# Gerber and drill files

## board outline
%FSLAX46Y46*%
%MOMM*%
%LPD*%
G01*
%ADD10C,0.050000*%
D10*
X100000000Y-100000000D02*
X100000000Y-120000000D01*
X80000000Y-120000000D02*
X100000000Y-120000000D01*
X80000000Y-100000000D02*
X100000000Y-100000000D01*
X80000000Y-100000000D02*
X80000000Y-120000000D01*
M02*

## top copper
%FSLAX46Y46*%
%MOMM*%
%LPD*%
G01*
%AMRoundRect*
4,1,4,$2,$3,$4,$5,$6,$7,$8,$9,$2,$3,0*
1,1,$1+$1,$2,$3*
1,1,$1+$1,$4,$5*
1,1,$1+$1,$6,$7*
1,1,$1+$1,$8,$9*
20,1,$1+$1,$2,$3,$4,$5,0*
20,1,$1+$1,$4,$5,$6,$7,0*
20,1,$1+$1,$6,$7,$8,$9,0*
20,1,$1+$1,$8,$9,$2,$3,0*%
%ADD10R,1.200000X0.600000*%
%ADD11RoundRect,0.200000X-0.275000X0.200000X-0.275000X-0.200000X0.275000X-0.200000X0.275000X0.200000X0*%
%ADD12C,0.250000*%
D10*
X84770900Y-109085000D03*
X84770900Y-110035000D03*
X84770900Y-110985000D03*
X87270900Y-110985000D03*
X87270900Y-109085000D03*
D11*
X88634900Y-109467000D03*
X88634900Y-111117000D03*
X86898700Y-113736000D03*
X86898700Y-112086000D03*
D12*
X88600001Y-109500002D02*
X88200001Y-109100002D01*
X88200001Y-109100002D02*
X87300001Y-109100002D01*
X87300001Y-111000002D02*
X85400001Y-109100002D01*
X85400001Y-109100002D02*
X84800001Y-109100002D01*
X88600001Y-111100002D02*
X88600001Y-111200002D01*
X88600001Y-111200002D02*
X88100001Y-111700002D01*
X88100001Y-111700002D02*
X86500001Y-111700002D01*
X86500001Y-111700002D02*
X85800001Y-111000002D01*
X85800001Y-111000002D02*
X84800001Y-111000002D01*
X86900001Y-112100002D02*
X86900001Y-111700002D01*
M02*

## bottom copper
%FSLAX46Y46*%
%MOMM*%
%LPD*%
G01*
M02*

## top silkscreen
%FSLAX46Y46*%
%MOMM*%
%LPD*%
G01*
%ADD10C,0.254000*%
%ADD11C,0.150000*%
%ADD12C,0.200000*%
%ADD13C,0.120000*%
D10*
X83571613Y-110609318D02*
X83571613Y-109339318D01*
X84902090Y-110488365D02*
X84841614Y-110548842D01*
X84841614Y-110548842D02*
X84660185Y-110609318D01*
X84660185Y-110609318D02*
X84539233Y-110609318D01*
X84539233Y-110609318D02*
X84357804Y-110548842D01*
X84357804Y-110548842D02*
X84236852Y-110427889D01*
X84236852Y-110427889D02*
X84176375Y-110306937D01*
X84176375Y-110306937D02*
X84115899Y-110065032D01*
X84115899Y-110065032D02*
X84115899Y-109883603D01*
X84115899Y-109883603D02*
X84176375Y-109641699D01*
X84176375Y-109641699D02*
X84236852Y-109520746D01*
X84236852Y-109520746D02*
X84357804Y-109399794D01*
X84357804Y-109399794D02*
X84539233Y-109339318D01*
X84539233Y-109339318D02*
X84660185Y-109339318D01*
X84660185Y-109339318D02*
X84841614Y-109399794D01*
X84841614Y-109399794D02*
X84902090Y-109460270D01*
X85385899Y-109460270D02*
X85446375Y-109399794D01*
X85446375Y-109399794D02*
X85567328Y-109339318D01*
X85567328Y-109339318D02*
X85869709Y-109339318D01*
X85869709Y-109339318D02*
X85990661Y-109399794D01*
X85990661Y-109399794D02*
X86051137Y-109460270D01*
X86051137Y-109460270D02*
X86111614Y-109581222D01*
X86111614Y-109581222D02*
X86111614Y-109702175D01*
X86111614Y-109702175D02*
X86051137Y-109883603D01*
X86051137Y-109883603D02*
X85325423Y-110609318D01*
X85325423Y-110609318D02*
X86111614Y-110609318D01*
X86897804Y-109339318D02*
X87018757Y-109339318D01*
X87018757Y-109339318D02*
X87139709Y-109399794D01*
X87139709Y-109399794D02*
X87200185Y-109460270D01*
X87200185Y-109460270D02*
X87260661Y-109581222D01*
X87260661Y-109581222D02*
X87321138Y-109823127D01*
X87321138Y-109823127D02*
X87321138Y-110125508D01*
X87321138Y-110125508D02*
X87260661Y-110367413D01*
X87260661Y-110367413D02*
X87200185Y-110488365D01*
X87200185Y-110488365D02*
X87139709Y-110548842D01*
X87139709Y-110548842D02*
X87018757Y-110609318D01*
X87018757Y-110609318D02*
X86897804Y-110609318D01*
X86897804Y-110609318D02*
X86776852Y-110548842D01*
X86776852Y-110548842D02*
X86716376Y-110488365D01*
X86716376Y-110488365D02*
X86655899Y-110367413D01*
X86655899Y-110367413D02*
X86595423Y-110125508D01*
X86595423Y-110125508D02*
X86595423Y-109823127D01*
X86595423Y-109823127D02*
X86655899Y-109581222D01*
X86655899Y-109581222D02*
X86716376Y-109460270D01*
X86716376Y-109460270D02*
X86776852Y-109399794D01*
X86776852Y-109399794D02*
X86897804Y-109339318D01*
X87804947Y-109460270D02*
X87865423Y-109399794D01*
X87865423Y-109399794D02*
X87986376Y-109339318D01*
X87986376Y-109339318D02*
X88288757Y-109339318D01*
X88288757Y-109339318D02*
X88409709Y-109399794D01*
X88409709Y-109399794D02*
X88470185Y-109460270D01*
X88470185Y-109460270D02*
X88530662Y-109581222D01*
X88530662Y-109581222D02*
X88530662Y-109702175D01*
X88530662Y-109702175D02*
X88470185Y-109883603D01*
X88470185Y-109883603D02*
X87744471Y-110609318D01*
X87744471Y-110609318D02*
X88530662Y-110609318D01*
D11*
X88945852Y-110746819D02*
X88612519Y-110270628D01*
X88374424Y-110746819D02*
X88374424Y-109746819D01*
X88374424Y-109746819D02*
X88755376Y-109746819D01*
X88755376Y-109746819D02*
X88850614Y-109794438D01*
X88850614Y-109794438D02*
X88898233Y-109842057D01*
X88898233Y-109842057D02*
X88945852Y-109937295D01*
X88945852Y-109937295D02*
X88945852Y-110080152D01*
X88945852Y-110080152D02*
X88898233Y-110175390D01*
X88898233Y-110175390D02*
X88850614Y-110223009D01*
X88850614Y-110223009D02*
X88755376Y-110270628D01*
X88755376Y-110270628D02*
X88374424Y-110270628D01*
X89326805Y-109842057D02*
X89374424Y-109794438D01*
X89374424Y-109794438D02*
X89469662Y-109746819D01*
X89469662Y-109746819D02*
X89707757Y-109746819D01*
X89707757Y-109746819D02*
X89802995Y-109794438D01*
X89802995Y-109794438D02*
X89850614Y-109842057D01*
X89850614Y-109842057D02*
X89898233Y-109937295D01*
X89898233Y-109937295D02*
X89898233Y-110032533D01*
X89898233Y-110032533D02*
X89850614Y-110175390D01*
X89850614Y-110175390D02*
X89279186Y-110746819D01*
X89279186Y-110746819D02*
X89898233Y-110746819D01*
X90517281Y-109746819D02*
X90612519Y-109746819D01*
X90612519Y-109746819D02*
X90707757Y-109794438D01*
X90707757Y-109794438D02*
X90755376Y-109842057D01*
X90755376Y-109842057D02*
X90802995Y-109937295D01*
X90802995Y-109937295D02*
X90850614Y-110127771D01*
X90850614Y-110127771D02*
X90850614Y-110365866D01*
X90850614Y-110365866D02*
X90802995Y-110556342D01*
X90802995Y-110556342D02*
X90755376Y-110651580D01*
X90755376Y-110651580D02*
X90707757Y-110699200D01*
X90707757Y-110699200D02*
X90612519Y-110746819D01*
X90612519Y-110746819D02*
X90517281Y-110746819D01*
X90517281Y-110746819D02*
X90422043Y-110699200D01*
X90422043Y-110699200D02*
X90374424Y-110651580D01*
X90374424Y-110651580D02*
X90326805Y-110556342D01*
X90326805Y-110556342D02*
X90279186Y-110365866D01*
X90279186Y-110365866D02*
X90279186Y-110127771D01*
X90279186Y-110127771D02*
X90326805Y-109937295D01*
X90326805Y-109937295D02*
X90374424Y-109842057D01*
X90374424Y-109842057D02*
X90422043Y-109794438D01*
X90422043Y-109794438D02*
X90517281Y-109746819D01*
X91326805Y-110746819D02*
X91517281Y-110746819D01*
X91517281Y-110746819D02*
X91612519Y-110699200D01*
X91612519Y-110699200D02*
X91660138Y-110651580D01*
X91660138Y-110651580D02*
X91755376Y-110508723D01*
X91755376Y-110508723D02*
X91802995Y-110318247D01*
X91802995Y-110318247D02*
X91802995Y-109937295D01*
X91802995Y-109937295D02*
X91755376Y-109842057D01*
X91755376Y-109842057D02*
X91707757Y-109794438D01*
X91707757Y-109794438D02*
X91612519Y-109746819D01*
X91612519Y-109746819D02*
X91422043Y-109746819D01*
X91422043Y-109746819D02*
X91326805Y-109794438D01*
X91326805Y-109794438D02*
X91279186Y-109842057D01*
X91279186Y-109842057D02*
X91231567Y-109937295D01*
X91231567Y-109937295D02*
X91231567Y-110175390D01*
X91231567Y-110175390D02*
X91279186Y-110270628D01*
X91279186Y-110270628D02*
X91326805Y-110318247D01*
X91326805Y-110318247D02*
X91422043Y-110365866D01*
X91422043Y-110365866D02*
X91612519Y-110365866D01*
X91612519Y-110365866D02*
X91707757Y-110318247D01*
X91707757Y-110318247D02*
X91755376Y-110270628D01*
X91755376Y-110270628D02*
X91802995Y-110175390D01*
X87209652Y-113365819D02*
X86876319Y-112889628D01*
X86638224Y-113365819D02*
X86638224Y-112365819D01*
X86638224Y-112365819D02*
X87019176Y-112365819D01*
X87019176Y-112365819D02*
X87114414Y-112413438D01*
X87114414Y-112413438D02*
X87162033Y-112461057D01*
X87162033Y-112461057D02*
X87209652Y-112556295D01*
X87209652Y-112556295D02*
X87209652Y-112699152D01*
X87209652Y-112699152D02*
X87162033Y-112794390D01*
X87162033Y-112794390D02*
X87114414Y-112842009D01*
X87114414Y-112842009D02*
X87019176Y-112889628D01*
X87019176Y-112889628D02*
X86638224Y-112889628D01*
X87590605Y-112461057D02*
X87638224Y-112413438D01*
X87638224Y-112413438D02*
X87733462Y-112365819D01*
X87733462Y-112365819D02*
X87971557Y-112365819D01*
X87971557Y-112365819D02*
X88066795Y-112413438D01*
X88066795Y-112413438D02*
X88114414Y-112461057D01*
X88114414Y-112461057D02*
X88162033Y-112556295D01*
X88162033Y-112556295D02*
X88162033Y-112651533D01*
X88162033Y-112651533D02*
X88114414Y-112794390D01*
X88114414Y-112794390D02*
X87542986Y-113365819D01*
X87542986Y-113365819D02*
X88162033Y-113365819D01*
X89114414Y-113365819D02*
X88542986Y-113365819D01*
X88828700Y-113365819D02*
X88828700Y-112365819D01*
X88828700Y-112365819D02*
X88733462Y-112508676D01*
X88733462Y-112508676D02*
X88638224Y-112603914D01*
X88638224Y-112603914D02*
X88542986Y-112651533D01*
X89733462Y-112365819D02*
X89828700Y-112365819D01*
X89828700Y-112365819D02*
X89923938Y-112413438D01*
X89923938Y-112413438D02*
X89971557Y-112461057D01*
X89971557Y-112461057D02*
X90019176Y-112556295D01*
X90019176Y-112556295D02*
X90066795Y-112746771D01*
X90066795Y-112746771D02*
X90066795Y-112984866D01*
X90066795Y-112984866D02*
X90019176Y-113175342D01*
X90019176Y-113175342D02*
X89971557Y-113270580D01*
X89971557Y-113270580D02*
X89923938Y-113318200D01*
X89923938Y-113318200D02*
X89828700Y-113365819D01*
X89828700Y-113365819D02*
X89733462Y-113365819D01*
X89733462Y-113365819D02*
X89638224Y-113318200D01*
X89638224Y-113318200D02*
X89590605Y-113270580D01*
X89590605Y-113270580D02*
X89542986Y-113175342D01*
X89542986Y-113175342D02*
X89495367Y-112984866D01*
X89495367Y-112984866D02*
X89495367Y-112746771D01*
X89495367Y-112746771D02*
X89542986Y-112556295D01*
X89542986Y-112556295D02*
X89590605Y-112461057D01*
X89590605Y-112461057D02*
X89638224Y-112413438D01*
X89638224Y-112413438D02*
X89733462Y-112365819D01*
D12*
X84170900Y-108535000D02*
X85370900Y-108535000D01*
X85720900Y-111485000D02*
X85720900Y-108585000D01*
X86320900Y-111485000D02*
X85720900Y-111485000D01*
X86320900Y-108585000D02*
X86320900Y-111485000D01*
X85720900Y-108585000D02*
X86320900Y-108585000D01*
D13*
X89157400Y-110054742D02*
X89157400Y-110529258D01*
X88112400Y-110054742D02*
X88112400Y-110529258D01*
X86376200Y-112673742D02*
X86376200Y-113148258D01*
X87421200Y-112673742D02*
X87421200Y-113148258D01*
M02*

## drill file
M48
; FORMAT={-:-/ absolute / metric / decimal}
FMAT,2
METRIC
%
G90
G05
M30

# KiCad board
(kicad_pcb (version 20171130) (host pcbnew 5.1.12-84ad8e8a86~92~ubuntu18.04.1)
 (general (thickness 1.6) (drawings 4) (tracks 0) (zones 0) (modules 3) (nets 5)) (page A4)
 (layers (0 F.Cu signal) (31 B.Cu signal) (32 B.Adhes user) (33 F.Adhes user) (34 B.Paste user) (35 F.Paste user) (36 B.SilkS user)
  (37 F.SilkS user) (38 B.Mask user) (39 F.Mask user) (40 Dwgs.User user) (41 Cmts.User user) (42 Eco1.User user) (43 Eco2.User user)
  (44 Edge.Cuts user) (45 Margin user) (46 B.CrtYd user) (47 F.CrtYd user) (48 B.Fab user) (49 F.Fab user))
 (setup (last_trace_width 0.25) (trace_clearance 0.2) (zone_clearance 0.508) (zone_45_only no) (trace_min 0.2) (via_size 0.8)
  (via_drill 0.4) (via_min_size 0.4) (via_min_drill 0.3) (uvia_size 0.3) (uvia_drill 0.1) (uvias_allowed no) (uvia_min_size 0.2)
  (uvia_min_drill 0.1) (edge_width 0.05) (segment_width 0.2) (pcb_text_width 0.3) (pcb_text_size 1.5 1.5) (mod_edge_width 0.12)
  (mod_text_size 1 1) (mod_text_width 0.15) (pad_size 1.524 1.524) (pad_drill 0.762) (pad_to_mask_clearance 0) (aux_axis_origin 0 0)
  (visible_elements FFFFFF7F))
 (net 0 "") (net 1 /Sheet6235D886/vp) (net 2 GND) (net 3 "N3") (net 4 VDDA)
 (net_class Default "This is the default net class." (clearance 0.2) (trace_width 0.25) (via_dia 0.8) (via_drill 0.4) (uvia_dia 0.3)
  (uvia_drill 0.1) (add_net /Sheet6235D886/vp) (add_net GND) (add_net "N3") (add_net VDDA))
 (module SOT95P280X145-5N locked (layer F.Cu) (at 86.020900 110.035000)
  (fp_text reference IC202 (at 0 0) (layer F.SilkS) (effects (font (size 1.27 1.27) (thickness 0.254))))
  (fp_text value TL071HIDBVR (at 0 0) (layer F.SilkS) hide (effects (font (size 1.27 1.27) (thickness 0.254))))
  (fp_line (start -1.85 -1.5) (end -0.65 -1.5) (layer F.SilkS) (width 0.2))
  (fp_line (start -0.3 1.45) (end -0.3 -1.45) (layer F.SilkS) (width 0.2))
  (fp_line (start 0.3 1.45) (end -0.3 1.45) (layer F.SilkS) (width 0.2))
  (fp_line (start 0.3 -1.45) (end 0.3 1.45) (layer F.SilkS) (width 0.2))
  (fp_line (start -0.3 -1.45) (end 0.3 -1.45) (layer F.SilkS) (width 0.2))
  (pad 1 smd rect (at -1.25 -0.95 90.000000) (size 0.6 1.2) (layers F.Cu F.Mask F.Paste) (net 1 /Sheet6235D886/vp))
  (pad 2 smd rect (at -1.25 0 90.000000) (size 0.6 1.2) (layers F.Cu F.Mask F.Paste) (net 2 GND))
  (pad 3 smd rect (at -1.25 0.95 90.000000) (size 0.6 1.2) (layers F.Cu F.Mask F.Paste) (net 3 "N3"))
  (pad 4 smd rect (at 1.25 0.95 90.000000) (size 0.6 1.2) (layers F.Cu F.Mask F.Paste) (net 1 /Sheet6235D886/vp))
  (pad 5 smd rect (at 1.25 -0.95 90.000000) (size 0.6 1.2) (layers F.Cu F.Mask F.Paste) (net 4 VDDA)))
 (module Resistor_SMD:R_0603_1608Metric (layer F.Cu) (at 88.634900 110.292000 270.000000)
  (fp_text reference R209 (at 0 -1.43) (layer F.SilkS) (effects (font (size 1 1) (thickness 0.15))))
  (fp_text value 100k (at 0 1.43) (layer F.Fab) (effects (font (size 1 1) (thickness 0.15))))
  (fp_line (start -0.237258 -0.5225) (end 0.237258 -0.5225) (layer F.SilkS) (width 0.12))
  (fp_line (start -0.237258 0.5225) (end 0.237258 0.5225) (layer F.SilkS) (width 0.12))
  (pad 1 smd roundrect (at -0.825 0 270.000000) (size 0.8 0.95) (layers F.Cu F.Mask F.Paste) (roundrect_rratio 0.25) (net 4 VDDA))
  (pad 2 smd roundrect (at 0.825 0 270.000000) (size 0.8 0.95) (layers F.Cu F.Mask F.Paste) (roundrect_rratio 0.25) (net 3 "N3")))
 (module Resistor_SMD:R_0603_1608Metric (layer F.Cu) (at 86.898700 112.911000 270.000000)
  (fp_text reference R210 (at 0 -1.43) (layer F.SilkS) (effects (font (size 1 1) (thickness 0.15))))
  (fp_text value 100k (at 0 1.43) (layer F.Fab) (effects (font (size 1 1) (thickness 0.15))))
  (fp_line (start -0.237258 0.5225) (end 0.237258 0.5225) (layer F.SilkS) (width 0.12))
  (fp_line (start -0.237258 -0.5225) (end 0.237258 -0.5225) (layer F.SilkS) (width 0.12))
  (pad 2 smd roundrect (at 0.825 0 270.000000) (size 0.8 0.95) (layers F.Cu F.Mask F.Paste) (roundrect_rratio 0.25) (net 2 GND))
  (pad 1 smd roundrect (at -0.825 0 270.000000) (size 0.8 0.95) (layers F.Cu F.Mask F.Paste) (roundrect_rratio 0.25) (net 3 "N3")))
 (gr_line (start 100 100) (end 100 120) (layer Edge.Cuts) (width 0.05))
 (gr_line (start 80 120) (end 100 120) (layer Edge.Cuts) (width 0.05))
 (gr_line (start 80 100) (end 100 100) (layer Edge.Cuts) (width 0.05))
 (gr_line (start 80 100) (end 80 120) (layer Edge.Cuts) (width 0.05))
 (segment (start 88.600001 109.500002) (end 88.200001 109.100002) (width 0.250000) (layer F.Cu) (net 4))
 (segment (start 88.200001 109.100002) (end 87.300001 109.100002) (width 0.250000) (layer F.Cu) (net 4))
 (segment (start 87.300001 111.000002) (end 85.400001 109.100002) (width 0.250000) (layer F.Cu) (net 1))
 (segment (start 85.400001 109.100002) (end 84.800001 109.100002) (width 0.250000) (layer F.Cu) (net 1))
 (segment (start 88.600001 111.100002) (end 88.600001 111.200002) (width 0.250000) (layer F.Cu) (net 3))
 (segment (start 88.600001 111.200002) (end 88.100001 111.700002) (width 0.250000) (layer F.Cu) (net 3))
 (segment (start 88.100001 111.700002) (end 86.500001 111.700002) (width 0.250000) (layer F.Cu) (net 3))
 (segment (start 86.500001 111.700002) (end 85.800001 111.000002) (width 0.250000) (layer F.Cu) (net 3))
 (segment (start 85.800001 111.000002) (end 84.800001 111.000002) (width 0.250000) (layer F.Cu) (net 3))
 (segment (start 86.900001 112.100002) (end 86.900001 111.700002) (width 0.250000) (layer F.Cu) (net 3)))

